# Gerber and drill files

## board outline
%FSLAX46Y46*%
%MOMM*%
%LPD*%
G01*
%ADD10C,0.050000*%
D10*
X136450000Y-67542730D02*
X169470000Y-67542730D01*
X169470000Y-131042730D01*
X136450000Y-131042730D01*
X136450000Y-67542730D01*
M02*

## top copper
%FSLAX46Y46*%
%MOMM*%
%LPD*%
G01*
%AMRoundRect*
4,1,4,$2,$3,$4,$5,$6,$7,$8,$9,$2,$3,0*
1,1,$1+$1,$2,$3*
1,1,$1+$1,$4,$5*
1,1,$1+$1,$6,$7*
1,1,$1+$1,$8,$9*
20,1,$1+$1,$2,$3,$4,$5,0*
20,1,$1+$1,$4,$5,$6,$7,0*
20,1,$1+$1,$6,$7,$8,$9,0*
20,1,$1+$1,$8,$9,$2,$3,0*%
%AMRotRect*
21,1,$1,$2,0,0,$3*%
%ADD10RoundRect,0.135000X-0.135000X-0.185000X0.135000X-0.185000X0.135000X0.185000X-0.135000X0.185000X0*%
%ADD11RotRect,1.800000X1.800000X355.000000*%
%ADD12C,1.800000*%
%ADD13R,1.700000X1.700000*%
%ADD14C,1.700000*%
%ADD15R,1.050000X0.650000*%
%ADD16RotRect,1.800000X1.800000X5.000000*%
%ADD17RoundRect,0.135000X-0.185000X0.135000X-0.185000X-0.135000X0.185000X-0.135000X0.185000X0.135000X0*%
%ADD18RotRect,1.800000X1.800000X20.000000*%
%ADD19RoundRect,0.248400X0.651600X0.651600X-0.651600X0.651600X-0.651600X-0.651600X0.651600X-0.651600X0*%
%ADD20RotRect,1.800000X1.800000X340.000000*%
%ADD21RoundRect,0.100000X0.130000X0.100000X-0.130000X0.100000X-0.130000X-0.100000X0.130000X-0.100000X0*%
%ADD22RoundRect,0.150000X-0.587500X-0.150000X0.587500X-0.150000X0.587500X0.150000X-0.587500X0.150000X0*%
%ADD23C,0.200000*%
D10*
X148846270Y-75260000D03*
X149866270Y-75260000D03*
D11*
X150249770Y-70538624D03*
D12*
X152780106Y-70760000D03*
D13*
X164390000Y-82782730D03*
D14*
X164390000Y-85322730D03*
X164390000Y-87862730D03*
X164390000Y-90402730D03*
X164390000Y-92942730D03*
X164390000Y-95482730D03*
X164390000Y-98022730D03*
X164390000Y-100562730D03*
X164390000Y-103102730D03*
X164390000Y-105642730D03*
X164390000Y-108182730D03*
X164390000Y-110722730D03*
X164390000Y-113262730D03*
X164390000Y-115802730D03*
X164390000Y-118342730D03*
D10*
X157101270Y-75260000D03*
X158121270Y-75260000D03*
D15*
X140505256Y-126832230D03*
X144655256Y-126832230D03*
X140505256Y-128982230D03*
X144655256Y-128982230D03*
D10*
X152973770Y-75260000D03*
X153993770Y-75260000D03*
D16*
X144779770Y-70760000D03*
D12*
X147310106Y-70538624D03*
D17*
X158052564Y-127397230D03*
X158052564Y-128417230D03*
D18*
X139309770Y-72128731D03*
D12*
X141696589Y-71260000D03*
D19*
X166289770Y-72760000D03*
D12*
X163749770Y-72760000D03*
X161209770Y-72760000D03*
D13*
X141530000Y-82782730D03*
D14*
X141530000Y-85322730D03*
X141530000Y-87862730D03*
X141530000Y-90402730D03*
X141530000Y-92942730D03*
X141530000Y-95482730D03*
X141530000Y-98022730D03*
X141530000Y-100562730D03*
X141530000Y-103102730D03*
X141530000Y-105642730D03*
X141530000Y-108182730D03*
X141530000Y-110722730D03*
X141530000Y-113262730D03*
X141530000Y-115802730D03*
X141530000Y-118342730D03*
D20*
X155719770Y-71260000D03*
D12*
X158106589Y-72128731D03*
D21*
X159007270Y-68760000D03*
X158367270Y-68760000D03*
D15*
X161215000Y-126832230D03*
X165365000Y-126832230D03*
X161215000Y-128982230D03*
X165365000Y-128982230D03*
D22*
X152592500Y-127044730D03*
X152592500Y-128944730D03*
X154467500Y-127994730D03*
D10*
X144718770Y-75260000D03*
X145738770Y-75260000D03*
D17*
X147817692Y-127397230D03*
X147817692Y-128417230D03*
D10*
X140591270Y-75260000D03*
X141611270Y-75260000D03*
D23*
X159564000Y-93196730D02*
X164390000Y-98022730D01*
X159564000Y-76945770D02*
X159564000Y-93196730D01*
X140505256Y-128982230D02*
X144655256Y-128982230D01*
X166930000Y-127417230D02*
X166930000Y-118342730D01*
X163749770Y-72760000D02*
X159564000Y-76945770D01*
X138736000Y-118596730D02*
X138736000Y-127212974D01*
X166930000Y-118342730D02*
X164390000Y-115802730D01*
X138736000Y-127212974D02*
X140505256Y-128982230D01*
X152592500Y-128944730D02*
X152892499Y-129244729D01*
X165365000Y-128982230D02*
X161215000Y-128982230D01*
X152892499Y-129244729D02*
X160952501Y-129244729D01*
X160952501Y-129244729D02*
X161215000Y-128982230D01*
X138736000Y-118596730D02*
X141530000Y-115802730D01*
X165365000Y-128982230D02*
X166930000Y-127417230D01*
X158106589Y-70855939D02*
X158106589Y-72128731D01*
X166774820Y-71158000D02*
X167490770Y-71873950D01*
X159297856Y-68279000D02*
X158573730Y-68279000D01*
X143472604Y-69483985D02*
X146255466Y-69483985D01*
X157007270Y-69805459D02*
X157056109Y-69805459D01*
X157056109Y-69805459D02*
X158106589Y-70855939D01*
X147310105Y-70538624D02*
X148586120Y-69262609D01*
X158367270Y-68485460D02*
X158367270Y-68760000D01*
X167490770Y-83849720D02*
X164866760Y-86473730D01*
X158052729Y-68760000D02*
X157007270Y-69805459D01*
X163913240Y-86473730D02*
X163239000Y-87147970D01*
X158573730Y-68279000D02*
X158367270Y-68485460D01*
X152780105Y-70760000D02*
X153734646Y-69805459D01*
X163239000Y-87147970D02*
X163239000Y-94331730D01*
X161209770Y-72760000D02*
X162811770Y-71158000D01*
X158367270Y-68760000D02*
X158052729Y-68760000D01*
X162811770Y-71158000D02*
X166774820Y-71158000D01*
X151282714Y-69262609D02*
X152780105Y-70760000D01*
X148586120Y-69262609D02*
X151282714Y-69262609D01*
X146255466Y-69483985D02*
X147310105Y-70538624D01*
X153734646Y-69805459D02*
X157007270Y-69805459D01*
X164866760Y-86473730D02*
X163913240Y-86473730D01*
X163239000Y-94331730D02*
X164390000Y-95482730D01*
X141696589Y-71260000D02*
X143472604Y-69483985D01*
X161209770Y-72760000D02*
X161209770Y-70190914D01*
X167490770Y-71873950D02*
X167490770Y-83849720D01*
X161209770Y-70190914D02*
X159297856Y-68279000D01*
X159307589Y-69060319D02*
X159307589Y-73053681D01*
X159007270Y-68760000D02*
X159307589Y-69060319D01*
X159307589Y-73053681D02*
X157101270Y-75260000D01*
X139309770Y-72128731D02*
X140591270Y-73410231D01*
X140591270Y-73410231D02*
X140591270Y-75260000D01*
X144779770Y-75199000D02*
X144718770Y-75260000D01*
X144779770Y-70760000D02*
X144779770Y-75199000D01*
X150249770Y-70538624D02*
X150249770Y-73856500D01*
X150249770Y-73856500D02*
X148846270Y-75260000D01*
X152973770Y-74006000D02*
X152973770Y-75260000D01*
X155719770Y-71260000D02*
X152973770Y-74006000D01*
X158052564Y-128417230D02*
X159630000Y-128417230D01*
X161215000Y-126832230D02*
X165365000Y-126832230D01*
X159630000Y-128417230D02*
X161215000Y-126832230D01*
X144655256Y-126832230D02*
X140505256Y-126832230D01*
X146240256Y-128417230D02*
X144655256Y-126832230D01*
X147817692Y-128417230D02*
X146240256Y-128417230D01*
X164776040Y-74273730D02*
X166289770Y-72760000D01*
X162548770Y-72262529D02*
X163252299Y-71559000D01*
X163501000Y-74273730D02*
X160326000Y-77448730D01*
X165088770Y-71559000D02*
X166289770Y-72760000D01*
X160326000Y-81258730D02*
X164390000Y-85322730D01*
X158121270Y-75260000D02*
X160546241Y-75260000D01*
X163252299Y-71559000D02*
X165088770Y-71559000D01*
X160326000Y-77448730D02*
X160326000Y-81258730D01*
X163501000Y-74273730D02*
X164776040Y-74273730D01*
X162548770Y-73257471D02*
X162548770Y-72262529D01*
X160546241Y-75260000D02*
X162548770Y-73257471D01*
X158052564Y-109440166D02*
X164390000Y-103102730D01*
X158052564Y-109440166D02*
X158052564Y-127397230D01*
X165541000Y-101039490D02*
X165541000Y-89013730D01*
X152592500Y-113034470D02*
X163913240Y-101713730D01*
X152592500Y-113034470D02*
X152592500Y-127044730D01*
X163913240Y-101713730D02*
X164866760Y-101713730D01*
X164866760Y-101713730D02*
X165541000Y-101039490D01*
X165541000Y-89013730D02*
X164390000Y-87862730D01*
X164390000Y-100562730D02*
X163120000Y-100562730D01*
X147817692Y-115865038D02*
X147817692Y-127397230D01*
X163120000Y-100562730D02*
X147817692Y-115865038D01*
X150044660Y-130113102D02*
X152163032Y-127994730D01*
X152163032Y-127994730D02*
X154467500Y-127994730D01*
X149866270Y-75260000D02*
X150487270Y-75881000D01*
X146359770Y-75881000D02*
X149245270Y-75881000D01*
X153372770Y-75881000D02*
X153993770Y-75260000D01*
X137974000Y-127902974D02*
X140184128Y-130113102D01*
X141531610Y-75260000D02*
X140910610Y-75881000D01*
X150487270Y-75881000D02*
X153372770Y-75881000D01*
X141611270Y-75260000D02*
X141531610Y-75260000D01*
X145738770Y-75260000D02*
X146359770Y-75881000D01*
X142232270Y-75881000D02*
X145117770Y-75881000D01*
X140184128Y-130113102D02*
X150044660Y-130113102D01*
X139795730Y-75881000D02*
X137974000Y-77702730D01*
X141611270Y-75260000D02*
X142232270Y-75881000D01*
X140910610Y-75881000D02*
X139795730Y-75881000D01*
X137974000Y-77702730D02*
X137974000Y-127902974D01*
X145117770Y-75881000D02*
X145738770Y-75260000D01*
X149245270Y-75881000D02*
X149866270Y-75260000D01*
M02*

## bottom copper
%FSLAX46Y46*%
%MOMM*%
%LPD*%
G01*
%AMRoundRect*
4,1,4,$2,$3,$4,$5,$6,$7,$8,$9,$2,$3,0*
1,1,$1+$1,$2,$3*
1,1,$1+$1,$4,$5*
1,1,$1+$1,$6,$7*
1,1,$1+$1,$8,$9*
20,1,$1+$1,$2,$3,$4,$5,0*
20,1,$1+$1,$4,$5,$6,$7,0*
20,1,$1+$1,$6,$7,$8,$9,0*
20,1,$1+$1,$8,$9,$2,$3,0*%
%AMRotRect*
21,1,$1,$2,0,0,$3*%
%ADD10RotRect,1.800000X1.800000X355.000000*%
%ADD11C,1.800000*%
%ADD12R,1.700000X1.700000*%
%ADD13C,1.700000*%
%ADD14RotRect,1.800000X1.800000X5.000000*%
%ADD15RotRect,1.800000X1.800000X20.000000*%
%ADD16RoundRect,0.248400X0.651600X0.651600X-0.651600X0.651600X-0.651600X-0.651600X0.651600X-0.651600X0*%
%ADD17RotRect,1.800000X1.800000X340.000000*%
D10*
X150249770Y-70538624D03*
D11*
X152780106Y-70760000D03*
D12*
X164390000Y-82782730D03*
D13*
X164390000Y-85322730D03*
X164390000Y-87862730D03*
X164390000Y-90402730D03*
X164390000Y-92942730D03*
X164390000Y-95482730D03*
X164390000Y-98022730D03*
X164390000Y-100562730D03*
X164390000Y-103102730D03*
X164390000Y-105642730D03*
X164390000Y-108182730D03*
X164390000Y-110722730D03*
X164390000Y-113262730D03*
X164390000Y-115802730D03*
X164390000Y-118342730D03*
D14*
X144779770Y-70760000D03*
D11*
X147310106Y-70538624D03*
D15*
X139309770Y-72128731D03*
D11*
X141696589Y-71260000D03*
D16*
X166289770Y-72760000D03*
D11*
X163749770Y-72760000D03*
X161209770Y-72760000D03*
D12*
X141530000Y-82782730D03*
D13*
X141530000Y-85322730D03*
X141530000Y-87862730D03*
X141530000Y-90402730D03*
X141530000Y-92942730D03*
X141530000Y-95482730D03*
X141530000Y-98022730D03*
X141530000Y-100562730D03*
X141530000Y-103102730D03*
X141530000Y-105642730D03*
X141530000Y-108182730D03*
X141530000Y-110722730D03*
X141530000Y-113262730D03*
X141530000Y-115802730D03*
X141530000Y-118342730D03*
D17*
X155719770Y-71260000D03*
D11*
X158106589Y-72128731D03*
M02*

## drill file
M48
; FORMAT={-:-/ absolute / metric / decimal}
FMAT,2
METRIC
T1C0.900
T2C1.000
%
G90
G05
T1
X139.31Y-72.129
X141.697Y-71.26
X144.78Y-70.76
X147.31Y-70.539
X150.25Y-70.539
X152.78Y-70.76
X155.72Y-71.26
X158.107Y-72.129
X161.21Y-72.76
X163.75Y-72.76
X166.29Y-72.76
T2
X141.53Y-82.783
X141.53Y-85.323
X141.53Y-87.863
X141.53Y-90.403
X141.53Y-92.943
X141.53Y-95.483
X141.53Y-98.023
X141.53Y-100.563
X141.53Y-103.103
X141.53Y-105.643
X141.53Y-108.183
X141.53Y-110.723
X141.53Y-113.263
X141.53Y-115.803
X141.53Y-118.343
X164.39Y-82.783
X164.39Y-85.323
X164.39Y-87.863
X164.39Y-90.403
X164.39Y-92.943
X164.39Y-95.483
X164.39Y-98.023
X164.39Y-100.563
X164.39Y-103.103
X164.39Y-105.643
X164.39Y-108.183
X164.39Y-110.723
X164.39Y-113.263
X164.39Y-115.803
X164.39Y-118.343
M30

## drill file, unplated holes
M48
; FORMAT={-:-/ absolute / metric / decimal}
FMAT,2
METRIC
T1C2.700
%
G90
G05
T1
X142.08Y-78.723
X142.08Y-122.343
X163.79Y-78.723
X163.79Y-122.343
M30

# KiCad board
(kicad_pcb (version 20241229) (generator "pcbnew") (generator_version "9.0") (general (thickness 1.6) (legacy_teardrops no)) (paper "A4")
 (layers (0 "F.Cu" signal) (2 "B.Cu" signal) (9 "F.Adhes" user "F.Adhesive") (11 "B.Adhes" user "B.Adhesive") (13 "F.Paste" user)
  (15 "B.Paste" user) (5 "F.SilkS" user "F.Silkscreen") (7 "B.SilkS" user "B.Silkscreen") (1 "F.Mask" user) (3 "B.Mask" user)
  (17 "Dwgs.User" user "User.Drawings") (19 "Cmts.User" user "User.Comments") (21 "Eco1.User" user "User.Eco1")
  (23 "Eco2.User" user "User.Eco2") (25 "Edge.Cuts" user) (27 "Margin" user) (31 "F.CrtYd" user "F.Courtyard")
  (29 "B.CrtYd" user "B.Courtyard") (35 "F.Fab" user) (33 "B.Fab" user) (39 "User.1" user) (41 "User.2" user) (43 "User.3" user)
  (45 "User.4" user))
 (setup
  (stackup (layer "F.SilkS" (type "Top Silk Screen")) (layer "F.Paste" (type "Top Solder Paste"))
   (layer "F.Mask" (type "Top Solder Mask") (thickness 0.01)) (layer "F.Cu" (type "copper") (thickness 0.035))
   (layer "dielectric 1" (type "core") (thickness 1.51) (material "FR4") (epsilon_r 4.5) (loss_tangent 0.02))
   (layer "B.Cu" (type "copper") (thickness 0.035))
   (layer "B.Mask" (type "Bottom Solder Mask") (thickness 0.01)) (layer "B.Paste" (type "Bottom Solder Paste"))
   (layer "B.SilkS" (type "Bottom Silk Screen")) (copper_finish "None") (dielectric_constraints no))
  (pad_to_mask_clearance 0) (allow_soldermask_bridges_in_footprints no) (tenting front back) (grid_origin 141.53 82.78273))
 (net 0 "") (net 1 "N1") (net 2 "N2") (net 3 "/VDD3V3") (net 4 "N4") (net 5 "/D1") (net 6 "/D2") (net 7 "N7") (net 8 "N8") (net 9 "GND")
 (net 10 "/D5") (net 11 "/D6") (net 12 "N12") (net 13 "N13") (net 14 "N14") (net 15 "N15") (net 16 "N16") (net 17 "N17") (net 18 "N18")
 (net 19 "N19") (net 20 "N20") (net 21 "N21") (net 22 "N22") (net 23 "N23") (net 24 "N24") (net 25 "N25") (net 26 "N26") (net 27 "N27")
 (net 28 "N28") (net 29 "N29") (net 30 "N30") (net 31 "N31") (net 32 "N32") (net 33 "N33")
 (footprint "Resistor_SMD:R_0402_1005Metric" (layer "F.Cu") (at 149.35627 75.26)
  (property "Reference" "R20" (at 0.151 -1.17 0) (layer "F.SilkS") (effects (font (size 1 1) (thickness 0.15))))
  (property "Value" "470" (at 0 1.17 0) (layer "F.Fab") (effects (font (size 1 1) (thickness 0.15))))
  (pad "1" smd roundrect (at -0.51 0) (size 0.54 0.64) (layers "F.Cu" "F.Mask" "F.Paste") (roundrect_rratio 0.25) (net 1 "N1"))
  (pad "2" smd roundrect (at 0.51 0) (size 0.54 0.64) (layers "F.Cu" "F.Mask" "F.Paste") (roundrect_rratio 0.25) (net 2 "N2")))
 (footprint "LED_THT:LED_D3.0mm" (layer "F.Cu") (at 150.24977 70.538624 -5)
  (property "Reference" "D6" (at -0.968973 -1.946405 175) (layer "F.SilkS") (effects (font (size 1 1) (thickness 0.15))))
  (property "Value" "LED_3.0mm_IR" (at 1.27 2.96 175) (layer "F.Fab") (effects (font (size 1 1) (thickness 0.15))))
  (pad "1" thru_hole rect (at 0 0 355) (size 1.8 1.8) (drill 0.9) (layers "*.Cu" "*.Mask") (remove_unused_layers no) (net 1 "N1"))
  (pad "2" thru_hole circle (at 2.540001 0 355) (size 1.8 1.8) (drill 0.9) (layers "*.Cu" "*.Mask") (remove_unused_layers no)
   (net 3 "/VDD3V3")))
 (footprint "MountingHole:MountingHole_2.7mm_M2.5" (layer "F.Cu") (at 142.08 78.72273)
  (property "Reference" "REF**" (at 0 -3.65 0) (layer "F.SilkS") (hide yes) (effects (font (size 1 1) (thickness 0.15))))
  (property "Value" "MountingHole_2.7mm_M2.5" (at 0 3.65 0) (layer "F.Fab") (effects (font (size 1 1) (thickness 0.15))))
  (pad "" np_thru_hole circle (at 0 0) (size 2.7 2.7) (drill 2.7) (layers "*.Cu" "*.Mask")))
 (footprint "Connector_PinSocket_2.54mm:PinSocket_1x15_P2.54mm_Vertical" (layer "F.Cu") (at 164.39 82.78273)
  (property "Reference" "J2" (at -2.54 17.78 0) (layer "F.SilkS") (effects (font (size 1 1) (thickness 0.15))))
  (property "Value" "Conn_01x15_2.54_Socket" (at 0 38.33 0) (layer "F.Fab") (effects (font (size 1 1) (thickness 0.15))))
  (pad "1" thru_hole rect (at 0 0) (size 1.7 1.7) (drill 1) (layers "*.Cu" "*.Mask") (remove_unused_layers no) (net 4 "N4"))
  (pad "2" thru_hole circle (at 0 2.54) (size 1.7 1.7) (drill 1) (layers "*.Cu" "*.Mask") (remove_unused_layers no) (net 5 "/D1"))
  (pad "3" thru_hole circle (at 0 5.08) (size 1.7 1.7) (drill 1) (layers "*.Cu" "*.Mask") (remove_unused_layers no) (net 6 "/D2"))
  (pad "4" thru_hole circle (at 0 7.62) (size 1.7 1.7) (drill 1) (layers "*.Cu" "*.Mask") (remove_unused_layers no) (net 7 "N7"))
  (pad "5" thru_hole circle (at 0 10.16) (size 1.7 1.7) (drill 1) (layers "*.Cu" "*.Mask") (remove_unused_layers no) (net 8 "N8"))
  (pad "6" thru_hole circle (at 0 12.7) (size 1.7 1.7) (drill 1) (layers "*.Cu" "*.Mask") (remove_unused_layers no) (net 3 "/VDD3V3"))
  (pad "7" thru_hole circle (at 0 15.24) (size 1.7 1.7) (drill 1) (layers "*.Cu" "*.Mask") (remove_unused_layers no) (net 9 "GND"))
  (pad "8" thru_hole circle (at 0 17.78) (size 1.7 1.7) (drill 1) (layers "*.Cu" "*.Mask") (remove_unused_layers no) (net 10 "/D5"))
  (pad "9" thru_hole circle (at 0 20.32) (size 1.7 1.7) (drill 1) (layers "*.Cu" "*.Mask") (remove_unused_layers no) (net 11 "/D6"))
  (pad "10" thru_hole circle (at 0 22.86) (size 1.7 1.7) (drill 1) (layers "*.Cu" "*.Mask") (remove_unused_layers no) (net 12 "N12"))
  (pad "11" thru_hole circle (at 0 25.4) (size 1.7 1.7) (drill 1) (layers "*.Cu" "*.Mask") (remove_unused_layers no) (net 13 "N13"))
  (pad "12" thru_hole circle (at 0 27.94) (size 1.7 1.7) (drill 1) (layers "*.Cu" "*.Mask") (remove_unused_layers no) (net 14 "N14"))
  (pad "13" thru_hole circle (at 0 30.48) (size 1.7 1.7) (drill 1) (layers "*.Cu" "*.Mask") (remove_unused_layers no) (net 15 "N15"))
  (pad "14" thru_hole circle (at 0 33.02) (size 1.7 1.7) (drill 1) (layers "*.Cu" "*.Mask") (remove_unused_layers no) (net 9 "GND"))
  (pad "15" thru_hole circle (at 0 35.56) (size 1.7 1.7) (drill 1) (layers "*.Cu" "*.Mask") (remove_unused_layers no) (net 3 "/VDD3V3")))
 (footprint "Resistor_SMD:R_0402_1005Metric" (layer "F.Cu") (at 157.61127 75.26)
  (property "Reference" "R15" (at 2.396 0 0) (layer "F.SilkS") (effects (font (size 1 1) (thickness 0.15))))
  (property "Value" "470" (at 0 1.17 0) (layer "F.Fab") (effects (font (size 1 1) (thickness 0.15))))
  (pad "1" smd roundrect (at -0.51 0) (size 0.54 0.64) (layers "F.Cu" "F.Mask" "F.Paste") (roundrect_rratio 0.25) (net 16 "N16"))
  (pad "2" smd roundrect (at 0.51 0) (size 0.54 0.64) (layers "F.Cu" "F.Mask" "F.Paste") (roundrect_rratio 0.25) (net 5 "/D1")))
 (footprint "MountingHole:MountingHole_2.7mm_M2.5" (layer "F.Cu") (at 163.79 122.34273)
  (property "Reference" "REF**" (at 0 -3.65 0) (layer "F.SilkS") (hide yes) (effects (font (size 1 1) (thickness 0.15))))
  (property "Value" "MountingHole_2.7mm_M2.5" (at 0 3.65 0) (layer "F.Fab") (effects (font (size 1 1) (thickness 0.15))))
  (pad "" np_thru_hole circle (at 0 0) (size 2.7 2.7) (drill 2.7) (layers "*.Cu" "*.Mask")))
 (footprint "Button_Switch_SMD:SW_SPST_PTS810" (layer "F.Cu") (at 142.580256 127.90723)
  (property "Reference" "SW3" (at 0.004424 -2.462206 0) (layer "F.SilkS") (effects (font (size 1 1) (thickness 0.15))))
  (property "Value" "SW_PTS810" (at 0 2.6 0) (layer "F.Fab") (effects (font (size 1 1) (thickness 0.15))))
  (pad "1" smd rect (at -2.075 -1.075) (size 1.05 0.65) (layers "F.Cu" "F.Mask" "F.Paste") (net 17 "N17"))
  (pad "1" smd rect (at 2.075 -1.075) (size 1.05 0.65) (layers "F.Cu" "F.Mask" "F.Paste") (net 17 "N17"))
  (pad "2" smd rect (at -2.075 1.075) (size 1.05 0.65) (layers "F.Cu" "F.Mask" "F.Paste") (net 9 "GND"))
  (pad "2" smd rect (at 2.075 1.075) (size 1.05 0.65) (layers "F.Cu" "F.Mask" "F.Paste") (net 9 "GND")))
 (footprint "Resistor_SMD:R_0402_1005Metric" (layer "F.Cu") (at 153.48377 75.26)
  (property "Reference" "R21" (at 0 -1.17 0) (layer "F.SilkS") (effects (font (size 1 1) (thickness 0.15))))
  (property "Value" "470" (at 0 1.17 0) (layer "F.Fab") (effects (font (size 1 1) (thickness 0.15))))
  (pad "1" smd roundrect (at -0.51 0) (size 0.54 0.64) (layers "F.Cu" "F.Mask" "F.Paste") (roundrect_rratio 0.25) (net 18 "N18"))
  (pad "2" smd roundrect (at 0.51 0) (size 0.54 0.64) (layers "F.Cu" "F.Mask" "F.Paste") (roundrect_rratio 0.25) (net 2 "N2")))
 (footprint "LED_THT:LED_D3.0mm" (layer "F.Cu") (at 144.77977 70.76 5)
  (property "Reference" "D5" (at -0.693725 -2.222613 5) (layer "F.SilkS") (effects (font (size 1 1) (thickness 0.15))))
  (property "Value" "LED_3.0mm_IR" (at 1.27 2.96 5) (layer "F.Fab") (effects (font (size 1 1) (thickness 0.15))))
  (pad "1" thru_hole rect (at 0 0 5) (size 1.8 1.8) (drill 0.9) (layers "*.Cu" "*.Mask") (remove_unused_layers no) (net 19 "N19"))
  (pad "2" thru_hole circle (at 2.540001 0 5) (size 1.8 1.8) (drill 0.9) (layers "*.Cu" "*.Mask") (remove_unused_layers no)
   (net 3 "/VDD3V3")))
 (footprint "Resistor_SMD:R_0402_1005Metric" (layer "F.Cu") (at 158.052564 127.90723 -90)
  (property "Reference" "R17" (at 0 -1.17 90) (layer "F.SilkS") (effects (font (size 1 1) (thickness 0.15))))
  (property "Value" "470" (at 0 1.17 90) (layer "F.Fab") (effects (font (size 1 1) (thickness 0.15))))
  (pad "1" smd roundrect (at -0.51 0 270) (size 0.54 0.64) (layers "F.Cu" "F.Mask" "F.Paste") (roundrect_rratio 0.25) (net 11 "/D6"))
  (pad "2" smd roundrect (at 0.51 0 270) (size 0.54 0.64) (layers "F.Cu" "F.Mask" "F.Paste") (roundrect_rratio 0.25) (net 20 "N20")))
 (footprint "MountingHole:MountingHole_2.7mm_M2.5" (layer "F.Cu") (at 163.79 78.72273)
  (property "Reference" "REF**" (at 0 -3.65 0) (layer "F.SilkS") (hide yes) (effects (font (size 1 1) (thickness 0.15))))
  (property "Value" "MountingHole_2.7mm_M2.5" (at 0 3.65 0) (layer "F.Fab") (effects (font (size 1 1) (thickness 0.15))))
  (pad "" np_thru_hole circle (at 0 0) (size 2.7 2.7) (drill 2.7) (layers "*.Cu" "*.Mask")))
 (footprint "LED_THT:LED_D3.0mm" (layer "F.Cu") (at 139.30977 72.128731 20)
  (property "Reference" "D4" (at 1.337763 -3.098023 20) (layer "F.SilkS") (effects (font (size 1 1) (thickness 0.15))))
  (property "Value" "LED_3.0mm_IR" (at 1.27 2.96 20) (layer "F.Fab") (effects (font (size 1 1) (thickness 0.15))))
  (pad "1" thru_hole rect (at 0 0 20) (size 1.8 1.8) (drill 0.9) (layers "*.Cu" "*.Mask") (remove_unused_layers no) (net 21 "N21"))
  (pad "2" thru_hole circle (at 2.54 0 20) (size 1.8 1.8) (drill 0.9) (layers "*.Cu" "*.Mask") (remove_unused_layers no) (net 3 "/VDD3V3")))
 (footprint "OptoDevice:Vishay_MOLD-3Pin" (layer "F.Cu") (at 166.28977 72.76 180)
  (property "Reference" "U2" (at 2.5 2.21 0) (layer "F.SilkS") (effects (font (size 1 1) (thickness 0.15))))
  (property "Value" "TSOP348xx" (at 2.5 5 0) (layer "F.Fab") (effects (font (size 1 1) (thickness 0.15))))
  (pad "1" thru_hole roundrect (at 0 0 180) (size 1.8 1.8) (drill 0.9) (layers "*.Cu" "*.Mask") (remove_unused_layers no)
   (roundrect_rratio 0.138) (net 5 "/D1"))
  (pad "2" thru_hole circle (at 2.54 0 180) (size 1.8 1.8) (drill 0.9) (layers "*.Cu" "*.Mask") (remove_unused_layers no) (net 9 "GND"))
  (pad "3" thru_hole circle (at 5.08 0 180) (size 1.8 1.8) (drill 0.9) (layers "*.Cu" "*.Mask") (remove_unused_layers no) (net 3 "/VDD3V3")))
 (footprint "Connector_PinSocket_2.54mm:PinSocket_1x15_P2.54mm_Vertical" (layer "F.Cu") (at 141.53 82.78273)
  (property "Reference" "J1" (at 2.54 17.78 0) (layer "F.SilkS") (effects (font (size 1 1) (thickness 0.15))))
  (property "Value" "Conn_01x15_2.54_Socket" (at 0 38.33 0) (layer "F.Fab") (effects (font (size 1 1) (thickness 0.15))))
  (pad "1" thru_hole rect (at 0 0) (size 1.7 1.7) (drill 1) (layers "*.Cu" "*.Mask") (remove_unused_layers no) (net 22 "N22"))
  (pad "2" thru_hole circle (at 0 2.54) (size 1.7 1.7) (drill 1) (layers "*.Cu" "*.Mask") (remove_unused_layers no) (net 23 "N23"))
  (pad "3" thru_hole circle (at 0 5.08) (size 1.7 1.7) (drill 1) (layers "*.Cu" "*.Mask") (remove_unused_layers no) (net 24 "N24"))
  (pad "4" thru_hole circle (at 0 7.62) (size 1.7 1.7) (drill 1) (layers "*.Cu" "*.Mask") (remove_unused_layers no) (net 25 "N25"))
  (pad "5" thru_hole circle (at 0 10.16) (size 1.7 1.7) (drill 1) (layers "*.Cu" "*.Mask") (remove_unused_layers no) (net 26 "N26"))
  (pad "6" thru_hole circle (at 0 12.7) (size 1.7 1.7) (drill 1) (layers "*.Cu" "*.Mask") (remove_unused_layers no) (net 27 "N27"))
  (pad "7" thru_hole circle (at 0 15.24) (size 1.7 1.7) (drill 1) (layers "*.Cu" "*.Mask") (remove_unused_layers no) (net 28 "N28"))
  (pad "8" thru_hole circle (at 0 17.78) (size 1.7 1.7) (drill 1) (layers "*.Cu" "*.Mask") (remove_unused_layers no) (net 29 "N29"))
  (pad "9" thru_hole circle (at 0 20.32) (size 1.7 1.7) (drill 1) (layers "*.Cu" "*.Mask") (remove_unused_layers no) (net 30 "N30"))
  (pad "10" thru_hole circle (at 0 22.86) (size 1.7 1.7) (drill 1) (layers "*.Cu" "*.Mask") (remove_unused_layers no) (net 9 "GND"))
  (pad "11" thru_hole circle (at 0 25.4) (size 1.7 1.7) (drill 1) (layers "*.Cu" "*.Mask") (remove_unused_layers no) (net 3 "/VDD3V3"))
  (pad "12" thru_hole circle (at 0 27.94) (size 1.7 1.7) (drill 1) (layers "*.Cu" "*.Mask") (remove_unused_layers no) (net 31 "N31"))
  (pad "13" thru_hole circle (at 0 30.48) (size 1.7 1.7) (drill 1) (layers "*.Cu" "*.Mask") (remove_unused_layers no) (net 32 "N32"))
  (pad "14" thru_hole circle (at 0 33.02) (size 1.7 1.7) (drill 1) (layers "*.Cu" "*.Mask") (remove_unused_layers no) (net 9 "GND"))
  (pad "15" thru_hole circle (at 0 35.56) (size 1.7 1.7) (drill 1) (layers "*.Cu" "*.Mask") (remove_unused_layers no) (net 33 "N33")))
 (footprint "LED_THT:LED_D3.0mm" (layer "F.Cu") (at 155.71977 71.26 -20)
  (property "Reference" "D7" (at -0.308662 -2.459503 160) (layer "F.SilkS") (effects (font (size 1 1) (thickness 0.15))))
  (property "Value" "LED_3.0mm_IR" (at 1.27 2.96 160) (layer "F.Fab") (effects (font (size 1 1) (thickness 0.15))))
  (pad "1" thru_hole rect (at 0 0 340) (size 1.8 1.8) (drill 0.9) (layers "*.Cu" "*.Mask") (remove_unused_layers no) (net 18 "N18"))
  (pad "2" thru_hole circle (at 2.54 0 340) (size 1.8 1.8) (drill 0.9) (layers "*.Cu" "*.Mask") (remove_unused_layers no) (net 3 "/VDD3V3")))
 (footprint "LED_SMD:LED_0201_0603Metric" (layer "F.Cu") (at 158.68727 68.76 180)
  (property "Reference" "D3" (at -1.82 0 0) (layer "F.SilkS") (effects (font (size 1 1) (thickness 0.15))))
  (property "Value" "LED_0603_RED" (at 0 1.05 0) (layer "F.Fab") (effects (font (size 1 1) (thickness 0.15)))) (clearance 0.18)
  (pad "" smd roundrect (at -0.345 0 180) (size 0.318 0.36) (layers "F.Paste") (roundrect_rratio 0.25))
  (pad "" smd roundrect (at 0.345 0 180) (size 0.318 0.36) (layers "F.Paste") (roundrect_rratio 0.25))
  (pad "1" smd roundrect (at -0.32 0 180) (size 0.46 0.4) (layers "F.Cu" "F.Mask") (roundrect_rratio 0.25) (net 16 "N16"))
  (pad "2" smd roundrect (at 0.32 0 180) (size 0.46 0.4) (layers "F.Cu" "F.Mask") (roundrect_rratio 0.25) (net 3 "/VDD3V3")))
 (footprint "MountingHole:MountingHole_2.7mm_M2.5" (layer "F.Cu") (at 142.08 122.34273)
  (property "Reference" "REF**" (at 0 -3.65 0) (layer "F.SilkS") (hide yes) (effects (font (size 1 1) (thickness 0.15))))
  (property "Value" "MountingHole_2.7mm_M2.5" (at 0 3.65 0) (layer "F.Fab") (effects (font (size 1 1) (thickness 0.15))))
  (pad "" np_thru_hole circle (at 0 0) (size 2.7 2.7) (drill 2.7) (layers "*.Cu" "*.Mask")))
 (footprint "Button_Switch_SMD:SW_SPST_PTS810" (layer "F.Cu") (at 163.29 127.90723)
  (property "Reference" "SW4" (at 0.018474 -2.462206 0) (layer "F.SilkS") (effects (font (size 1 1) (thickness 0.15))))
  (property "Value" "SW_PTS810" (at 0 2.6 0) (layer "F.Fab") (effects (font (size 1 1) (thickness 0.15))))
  (pad "1" smd rect (at -2.075 -1.075) (size 1.05 0.65) (layers "F.Cu" "F.Mask" "F.Paste") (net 20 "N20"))
  (pad "1" smd rect (at 2.075 -1.075) (size 1.05 0.65) (layers "F.Cu" "F.Mask" "F.Paste") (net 20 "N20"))
  (pad "2" smd rect (at -2.075 1.075) (size 1.05 0.65) (layers "F.Cu" "F.Mask" "F.Paste") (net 9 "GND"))
  (pad "2" smd rect (at 2.075 1.075) (size 1.05 0.65) (layers "F.Cu" "F.Mask" "F.Paste") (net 9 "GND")))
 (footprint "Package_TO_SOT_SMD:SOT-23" (layer "F.Cu") (at 153.53 127.99473)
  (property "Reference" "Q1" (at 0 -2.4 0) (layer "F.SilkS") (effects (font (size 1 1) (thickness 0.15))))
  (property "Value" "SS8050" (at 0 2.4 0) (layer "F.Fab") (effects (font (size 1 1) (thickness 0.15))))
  (pad "1" smd roundrect (at -0.9375 -0.95) (size 1.475 0.6) (layers "F.Cu" "F.Mask" "F.Paste") (roundrect_rratio 0.25) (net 6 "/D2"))
  (pad "2" smd roundrect (at -0.9375 0.95) (size 1.475 0.6) (layers "F.Cu" "F.Mask" "F.Paste") (roundrect_rratio 0.25) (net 9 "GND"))
  (pad "3" smd roundrect (at 0.9375 0) (size 1.475 0.6) (layers "F.Cu" "F.Mask" "F.Paste") (roundrect_rratio 0.25) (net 2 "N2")))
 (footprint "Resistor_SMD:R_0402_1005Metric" (layer "F.Cu") (at 145.22877 75.26)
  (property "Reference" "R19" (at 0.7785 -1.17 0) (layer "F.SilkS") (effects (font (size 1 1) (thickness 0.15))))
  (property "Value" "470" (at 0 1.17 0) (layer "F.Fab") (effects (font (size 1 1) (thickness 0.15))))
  (pad "1" smd roundrect (at -0.51 0) (size 0.54 0.64) (layers "F.Cu" "F.Mask" "F.Paste") (roundrect_rratio 0.25) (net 19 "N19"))
  (pad "2" smd roundrect (at 0.51 0) (size 0.54 0.64) (layers "F.Cu" "F.Mask" "F.Paste") (roundrect_rratio 0.25) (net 2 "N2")))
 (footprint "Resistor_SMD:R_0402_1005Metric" (layer "F.Cu") (at 147.817692 127.90723 -90)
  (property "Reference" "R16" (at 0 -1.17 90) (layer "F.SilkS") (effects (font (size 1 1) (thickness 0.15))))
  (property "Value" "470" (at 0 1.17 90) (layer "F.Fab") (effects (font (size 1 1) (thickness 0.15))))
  (pad "1" smd roundrect (at -0.51 0 270) (size 0.54 0.64) (layers "F.Cu" "F.Mask" "F.Paste") (roundrect_rratio 0.25) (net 10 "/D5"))
  (pad "2" smd roundrect (at 0.51 0 270) (size 0.54 0.64) (layers "F.Cu" "F.Mask" "F.Paste") (roundrect_rratio 0.25) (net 17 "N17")))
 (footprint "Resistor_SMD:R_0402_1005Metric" (layer "F.Cu") (at 141.10127 75.26)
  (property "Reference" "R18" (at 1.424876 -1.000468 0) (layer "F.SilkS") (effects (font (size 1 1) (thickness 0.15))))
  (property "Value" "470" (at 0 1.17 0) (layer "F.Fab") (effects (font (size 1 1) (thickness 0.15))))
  (pad "1" smd roundrect (at -0.51 0) (size 0.54 0.64) (layers "F.Cu" "F.Mask" "F.Paste") (roundrect_rratio 0.25) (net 21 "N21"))
  (pad "2" smd roundrect (at 0.51 0) (size 0.54 0.64) (layers "F.Cu" "F.Mask" "F.Paste") (roundrect_rratio 0.25) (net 2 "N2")))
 (gr_rect (start 136.45 67.54273) (end 169.47 131.04273) (stroke (width 0.05) (type default)) (fill no) (layer "Edge.Cuts"))
 (segment (start 159.564 93.19673) (end 164.39 98.02273) (width 0.2) (layer "F.Cu") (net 9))
 (segment (start 159.564 76.94577) (end 159.564 93.19673) (width 0.2) (layer "F.Cu") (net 9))
 (segment (start 140.505256 128.98223) (end 144.655256 128.98223) (width 0.2) (layer "F.Cu") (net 9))
 (segment (start 166.93 127.41723) (end 166.93 118.34273) (width 0.2) (layer "F.Cu") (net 9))
 (segment (start 163.74977 72.76) (end 159.564 76.94577) (width 0.2) (layer "F.Cu") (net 9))
 (segment (start 138.736 118.59673) (end 138.736 127.212974) (width 0.2) (layer "F.Cu") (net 9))
 (segment (start 166.93 118.34273) (end 164.39 115.80273) (width 0.2) (layer "F.Cu") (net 9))
 (segment (start 138.736 127.212974) (end 140.505256 128.98223) (width 0.2) (layer "F.Cu") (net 9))
 (segment (start 152.5925 128.94473) (end 152.892499 129.244729) (width 0.2) (layer "F.Cu") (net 9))
 (segment (start 165.365 128.98223) (end 161.215 128.98223) (width 0.2) (layer "F.Cu") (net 9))
 (segment (start 152.892499 129.244729) (end 160.952501 129.244729) (width 0.2) (layer "F.Cu") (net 9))
 (segment (start 160.952501 129.244729) (end 161.215 128.98223) (width 0.2) (layer "F.Cu") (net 9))
 (segment (start 138.736 118.59673) (end 141.53 115.80273) (width 0.2) (layer "F.Cu") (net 9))
 (segment (start 165.365 128.98223) (end 166.93 127.41723) (width 0.2) (layer "F.Cu") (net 9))
 (segment (start 158.106589 70.855939) (end 158.106589 72.128731) (width 0.2) (layer "F.Cu") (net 3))
 (segment (start 166.77482 71.158) (end 167.49077 71.87395) (width 0.2) (layer "F.Cu") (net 3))
 (segment (start 159.297856 68.279) (end 158.57373 68.279) (width 0.2) (layer "F.Cu") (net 3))
 (segment (start 143.472604 69.483985) (end 146.255466 69.483985) (width 0.2) (layer "F.Cu") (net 3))
 (segment (start 157.00727 69.805459) (end 157.056109 69.805459) (width 0.2) (layer "F.Cu") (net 3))
 (segment (start 157.056109 69.805459) (end 158.106589 70.855939) (width 0.2) (layer "F.Cu") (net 3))
 (segment (start 147.310105 70.538624) (end 148.58612 69.262609) (width 0.2) (layer "F.Cu") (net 3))
 (segment (start 158.36727 68.48546) (end 158.36727 68.76) (width 0.2) (layer "F.Cu") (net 3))
 (segment (start 167.49077 83.84972) (end 164.86676 86.47373) (width 0.2) (layer "F.Cu") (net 3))
 (segment (start 158.052729 68.76) (end 157.00727 69.805459) (width 0.2) (layer "F.Cu") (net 3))
 (segment (start 163.91324 86.47373) (end 163.239 87.14797) (width 0.2) (layer "F.Cu") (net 3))
 (segment (start 158.57373 68.279) (end 158.36727 68.48546) (width 0.2) (layer "F.Cu") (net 3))
 (segment (start 152.780105 70.76) (end 153.734646 69.805459) (width 0.2) (layer "F.Cu") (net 3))
 (segment (start 163.239 87.14797) (end 163.239 94.33173) (width 0.2) (layer "F.Cu") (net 3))
 (segment (start 161.20977 72.76) (end 162.81177 71.158) (width 0.2) (layer "F.Cu") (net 3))
 (segment (start 158.36727 68.76) (end 158.052729 68.76) (width 0.2) (layer "F.Cu") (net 3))
 (segment (start 162.81177 71.158) (end 166.77482 71.158) (width 0.2) (layer "F.Cu") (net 3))
 (segment (start 151.282714 69.262609) (end 152.780105 70.76) (width 0.2) (layer "F.Cu") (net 3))
 (segment (start 148.58612 69.262609) (end 151.282714 69.262609) (width 0.2) (layer "F.Cu") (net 3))
 (segment (start 146.255466 69.483985) (end 147.310105 70.538624) (width 0.2) (layer "F.Cu") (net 3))
 (segment (start 153.734646 69.805459) (end 157.00727 69.805459) (width 0.2) (layer "F.Cu") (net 3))
 (segment (start 164.86676 86.47373) (end 163.91324 86.47373) (width 0.2) (layer "F.Cu") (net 3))
 (segment (start 163.239 94.33173) (end 164.39 95.48273) (width 0.2) (layer "F.Cu") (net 3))
 (segment (start 141.696589 71.26) (end 143.472604 69.483985) (width 0.2) (layer "F.Cu") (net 3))
 (segment (start 161.20977 72.76) (end 161.20977 70.190914) (width 0.2) (layer "F.Cu") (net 3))
 (segment (start 167.49077 71.87395) (end 167.49077 83.84972) (width 0.2) (layer "F.Cu") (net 3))
 (segment (start 161.20977 70.190914) (end 159.297856 68.279) (width 0.2) (layer "F.Cu") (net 3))
 (segment (start 159.307589 69.060319) (end 159.307589 73.053681) (width 0.2) (layer "F.Cu") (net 16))
 (segment (start 159.00727 68.76) (end 159.307589 69.060319) (width 0.2) (layer "F.Cu") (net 16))
 (segment (start 159.307589 73.053681) (end 157.10127 75.26) (width 0.2) (layer "F.Cu") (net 16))
 (segment (start 139.30977 72.128731) (end 140.59127 73.410231) (width 0.2) (layer "F.Cu") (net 21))
 (segment (start 140.59127 73.410231) (end 140.59127 75.26) (width 0.2) (layer "F.Cu") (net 21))
 (segment (start 144.77977 75.199) (end 144.71877 75.26) (width 0.2) (layer "F.Cu") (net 19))
 (segment (start 144.77977 70.76) (end 144.77977 75.199) (width 0.2) (layer "F.Cu") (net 19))
 (segment (start 150.24977 70.538624) (end 150.24977 73.8565) (width 0.2) (layer "F.Cu") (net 1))
 (segment (start 150.24977 73.8565) (end 148.84627 75.26) (width 0.2) (layer "F.Cu") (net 1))
 (segment (start 152.97377 74.006) (end 152.97377 75.26) (width 0.2) (layer "F.Cu") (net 18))
 (segment (start 155.71977 71.26) (end 152.97377 74.006) (width 0.2) (layer "F.Cu") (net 18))
 (segment (start 158.052564 128.41723) (end 159.63 128.41723) (width 0.2) (layer "F.Cu") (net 20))
 (segment (start 161.215 126.83223) (end 165.365 126.83223) (width 0.2) (layer "F.Cu") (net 20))
 (segment (start 159.63 128.41723) (end 161.215 126.83223) (width 0.2) (layer "F.Cu") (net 20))
 (segment (start 144.655256 126.83223) (end 140.505256 126.83223) (width 0.2) (layer "F.Cu") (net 17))
 (segment (start 146.240256 128.41723) (end 144.655256 126.83223) (width 0.2) (layer "F.Cu") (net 17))
 (segment (start 147.817692 128.41723) (end 146.240256 128.41723) (width 0.2) (layer "F.Cu") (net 17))
 (segment (start 164.77604 74.27373) (end 166.28977 72.76) (width 0.2) (layer "F.Cu") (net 5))
 (segment (start 162.54877 72.262529) (end 163.252299 71.559) (width 0.2) (layer "F.Cu") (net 5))
 (segment (start 163.501 74.27373) (end 160.326 77.44873) (width 0.2) (layer "F.Cu") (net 5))
 (segment (start 165.08877 71.559) (end 166.28977 72.76) (width 0.2) (layer "F.Cu") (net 5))
 (segment (start 160.326 81.25873) (end 164.39 85.32273) (width 0.2) (layer "F.Cu") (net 5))
 (segment (start 158.12127 75.26) (end 160.546241 75.26) (width 0.2) (layer "F.Cu") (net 5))
 (segment (start 163.252299 71.559) (end 165.08877 71.559) (width 0.2) (layer "F.Cu") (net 5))
 (segment (start 160.326 77.44873) (end 160.326 81.25873) (width 0.2) (layer "F.Cu") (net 5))
 (segment (start 163.501 74.27373) (end 164.77604 74.27373) (width 0.2) (layer "F.Cu") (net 5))
 (segment (start 162.54877 73.257471) (end 162.54877 72.262529) (width 0.2) (layer "F.Cu") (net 5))
 (segment (start 160.546241 75.26) (end 162.54877 73.257471) (width 0.2) (layer "F.Cu") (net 5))
 (segment (start 158.052564 109.440166) (end 164.39 103.10273) (width 0.2) (layer "F.Cu") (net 11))
 (segment (start 158.052564 109.440166) (end 158.052564 127.39723) (width 0.2) (layer "F.Cu") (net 11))
 (segment (start 165.541 101.03949) (end 165.541 89.01373) (width 0.2) (layer "F.Cu") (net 6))
 (segment (start 152.5925 113.03447) (end 163.91324 101.71373) (width 0.2) (layer "F.Cu") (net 6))
 (segment (start 152.5925 113.03447) (end 152.5925 127.04473) (width 0.2) (layer "F.Cu") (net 6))
 (segment (start 163.91324 101.71373) (end 164.86676 101.71373) (width 0.2) (layer "F.Cu") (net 6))
 (segment (start 164.86676 101.71373) (end 165.541 101.03949) (width 0.2) (layer "F.Cu") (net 6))
 (segment (start 165.541 89.01373) (end 164.39 87.86273) (width 0.2) (layer "F.Cu") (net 6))
 (segment (start 164.39 100.56273) (end 163.12 100.56273) (width 0.2) (layer "F.Cu") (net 10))
 (segment (start 147.817692 115.865038) (end 147.817692 127.39723) (width 0.2) (layer "F.Cu") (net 10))
 (segment (start 163.12 100.56273) (end 147.817692 115.865038) (width 0.2) (layer "F.Cu") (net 10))
 (segment (start 150.04466 130.113102) (end 152.163032 127.99473) (width 0.2) (layer "F.Cu") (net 2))
 (segment (start 152.163032 127.99473) (end 154.4675 127.99473) (width 0.2) (layer "F.Cu") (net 2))
 (segment (start 149.86627 75.26) (end 150.48727 75.881) (width 0.2) (layer "F.Cu") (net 2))
 (segment (start 146.35977 75.881) (end 149.24527 75.881) (width 0.2) (layer "F.Cu") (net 2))
 (segment (start 153.37277 75.881) (end 153.99377 75.26) (width 0.2) (layer "F.Cu") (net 2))
 (segment (start 137.974 127.902974) (end 140.184128 130.113102) (width 0.2) (layer "F.Cu") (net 2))
 (segment (start 141.53161 75.26) (end 140.91061 75.881) (width 0.2) (layer "F.Cu") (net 2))
 (segment (start 150.48727 75.881) (end 153.37277 75.881) (width 0.2) (layer "F.Cu") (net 2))
 (segment (start 141.61127 75.26) (end 141.53161 75.26) (width 0.2) (layer "F.Cu") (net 2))
 (segment (start 145.73877 75.26) (end 146.35977 75.881) (width 0.2) (layer "F.Cu") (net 2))
 (segment (start 142.23227 75.881) (end 145.11777 75.881) (width 0.2) (layer "F.Cu") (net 2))
 (segment (start 140.184128 130.113102) (end 150.04466 130.113102) (width 0.2) (layer "F.Cu") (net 2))
 (segment (start 139.79573 75.881) (end 137.974 77.70273) (width 0.2) (layer "F.Cu") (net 2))
 (segment (start 141.61127 75.26) (end 142.23227 75.881) (width 0.2) (layer "F.Cu") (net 2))
 (segment (start 140.91061 75.881) (end 139.79573 75.881) (width 0.2) (layer "F.Cu") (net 2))
 (segment (start 137.974 77.70273) (end 137.974 127.902974) (width 0.2) (layer "F.Cu") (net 2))
 (segment (start 145.11777 75.881) (end 145.73877 75.26) (width 0.2) (layer "F.Cu") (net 2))
 (segment (start 149.24527 75.881) (end 149.86627 75.26) (width 0.2) (layer "F.Cu") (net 2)))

